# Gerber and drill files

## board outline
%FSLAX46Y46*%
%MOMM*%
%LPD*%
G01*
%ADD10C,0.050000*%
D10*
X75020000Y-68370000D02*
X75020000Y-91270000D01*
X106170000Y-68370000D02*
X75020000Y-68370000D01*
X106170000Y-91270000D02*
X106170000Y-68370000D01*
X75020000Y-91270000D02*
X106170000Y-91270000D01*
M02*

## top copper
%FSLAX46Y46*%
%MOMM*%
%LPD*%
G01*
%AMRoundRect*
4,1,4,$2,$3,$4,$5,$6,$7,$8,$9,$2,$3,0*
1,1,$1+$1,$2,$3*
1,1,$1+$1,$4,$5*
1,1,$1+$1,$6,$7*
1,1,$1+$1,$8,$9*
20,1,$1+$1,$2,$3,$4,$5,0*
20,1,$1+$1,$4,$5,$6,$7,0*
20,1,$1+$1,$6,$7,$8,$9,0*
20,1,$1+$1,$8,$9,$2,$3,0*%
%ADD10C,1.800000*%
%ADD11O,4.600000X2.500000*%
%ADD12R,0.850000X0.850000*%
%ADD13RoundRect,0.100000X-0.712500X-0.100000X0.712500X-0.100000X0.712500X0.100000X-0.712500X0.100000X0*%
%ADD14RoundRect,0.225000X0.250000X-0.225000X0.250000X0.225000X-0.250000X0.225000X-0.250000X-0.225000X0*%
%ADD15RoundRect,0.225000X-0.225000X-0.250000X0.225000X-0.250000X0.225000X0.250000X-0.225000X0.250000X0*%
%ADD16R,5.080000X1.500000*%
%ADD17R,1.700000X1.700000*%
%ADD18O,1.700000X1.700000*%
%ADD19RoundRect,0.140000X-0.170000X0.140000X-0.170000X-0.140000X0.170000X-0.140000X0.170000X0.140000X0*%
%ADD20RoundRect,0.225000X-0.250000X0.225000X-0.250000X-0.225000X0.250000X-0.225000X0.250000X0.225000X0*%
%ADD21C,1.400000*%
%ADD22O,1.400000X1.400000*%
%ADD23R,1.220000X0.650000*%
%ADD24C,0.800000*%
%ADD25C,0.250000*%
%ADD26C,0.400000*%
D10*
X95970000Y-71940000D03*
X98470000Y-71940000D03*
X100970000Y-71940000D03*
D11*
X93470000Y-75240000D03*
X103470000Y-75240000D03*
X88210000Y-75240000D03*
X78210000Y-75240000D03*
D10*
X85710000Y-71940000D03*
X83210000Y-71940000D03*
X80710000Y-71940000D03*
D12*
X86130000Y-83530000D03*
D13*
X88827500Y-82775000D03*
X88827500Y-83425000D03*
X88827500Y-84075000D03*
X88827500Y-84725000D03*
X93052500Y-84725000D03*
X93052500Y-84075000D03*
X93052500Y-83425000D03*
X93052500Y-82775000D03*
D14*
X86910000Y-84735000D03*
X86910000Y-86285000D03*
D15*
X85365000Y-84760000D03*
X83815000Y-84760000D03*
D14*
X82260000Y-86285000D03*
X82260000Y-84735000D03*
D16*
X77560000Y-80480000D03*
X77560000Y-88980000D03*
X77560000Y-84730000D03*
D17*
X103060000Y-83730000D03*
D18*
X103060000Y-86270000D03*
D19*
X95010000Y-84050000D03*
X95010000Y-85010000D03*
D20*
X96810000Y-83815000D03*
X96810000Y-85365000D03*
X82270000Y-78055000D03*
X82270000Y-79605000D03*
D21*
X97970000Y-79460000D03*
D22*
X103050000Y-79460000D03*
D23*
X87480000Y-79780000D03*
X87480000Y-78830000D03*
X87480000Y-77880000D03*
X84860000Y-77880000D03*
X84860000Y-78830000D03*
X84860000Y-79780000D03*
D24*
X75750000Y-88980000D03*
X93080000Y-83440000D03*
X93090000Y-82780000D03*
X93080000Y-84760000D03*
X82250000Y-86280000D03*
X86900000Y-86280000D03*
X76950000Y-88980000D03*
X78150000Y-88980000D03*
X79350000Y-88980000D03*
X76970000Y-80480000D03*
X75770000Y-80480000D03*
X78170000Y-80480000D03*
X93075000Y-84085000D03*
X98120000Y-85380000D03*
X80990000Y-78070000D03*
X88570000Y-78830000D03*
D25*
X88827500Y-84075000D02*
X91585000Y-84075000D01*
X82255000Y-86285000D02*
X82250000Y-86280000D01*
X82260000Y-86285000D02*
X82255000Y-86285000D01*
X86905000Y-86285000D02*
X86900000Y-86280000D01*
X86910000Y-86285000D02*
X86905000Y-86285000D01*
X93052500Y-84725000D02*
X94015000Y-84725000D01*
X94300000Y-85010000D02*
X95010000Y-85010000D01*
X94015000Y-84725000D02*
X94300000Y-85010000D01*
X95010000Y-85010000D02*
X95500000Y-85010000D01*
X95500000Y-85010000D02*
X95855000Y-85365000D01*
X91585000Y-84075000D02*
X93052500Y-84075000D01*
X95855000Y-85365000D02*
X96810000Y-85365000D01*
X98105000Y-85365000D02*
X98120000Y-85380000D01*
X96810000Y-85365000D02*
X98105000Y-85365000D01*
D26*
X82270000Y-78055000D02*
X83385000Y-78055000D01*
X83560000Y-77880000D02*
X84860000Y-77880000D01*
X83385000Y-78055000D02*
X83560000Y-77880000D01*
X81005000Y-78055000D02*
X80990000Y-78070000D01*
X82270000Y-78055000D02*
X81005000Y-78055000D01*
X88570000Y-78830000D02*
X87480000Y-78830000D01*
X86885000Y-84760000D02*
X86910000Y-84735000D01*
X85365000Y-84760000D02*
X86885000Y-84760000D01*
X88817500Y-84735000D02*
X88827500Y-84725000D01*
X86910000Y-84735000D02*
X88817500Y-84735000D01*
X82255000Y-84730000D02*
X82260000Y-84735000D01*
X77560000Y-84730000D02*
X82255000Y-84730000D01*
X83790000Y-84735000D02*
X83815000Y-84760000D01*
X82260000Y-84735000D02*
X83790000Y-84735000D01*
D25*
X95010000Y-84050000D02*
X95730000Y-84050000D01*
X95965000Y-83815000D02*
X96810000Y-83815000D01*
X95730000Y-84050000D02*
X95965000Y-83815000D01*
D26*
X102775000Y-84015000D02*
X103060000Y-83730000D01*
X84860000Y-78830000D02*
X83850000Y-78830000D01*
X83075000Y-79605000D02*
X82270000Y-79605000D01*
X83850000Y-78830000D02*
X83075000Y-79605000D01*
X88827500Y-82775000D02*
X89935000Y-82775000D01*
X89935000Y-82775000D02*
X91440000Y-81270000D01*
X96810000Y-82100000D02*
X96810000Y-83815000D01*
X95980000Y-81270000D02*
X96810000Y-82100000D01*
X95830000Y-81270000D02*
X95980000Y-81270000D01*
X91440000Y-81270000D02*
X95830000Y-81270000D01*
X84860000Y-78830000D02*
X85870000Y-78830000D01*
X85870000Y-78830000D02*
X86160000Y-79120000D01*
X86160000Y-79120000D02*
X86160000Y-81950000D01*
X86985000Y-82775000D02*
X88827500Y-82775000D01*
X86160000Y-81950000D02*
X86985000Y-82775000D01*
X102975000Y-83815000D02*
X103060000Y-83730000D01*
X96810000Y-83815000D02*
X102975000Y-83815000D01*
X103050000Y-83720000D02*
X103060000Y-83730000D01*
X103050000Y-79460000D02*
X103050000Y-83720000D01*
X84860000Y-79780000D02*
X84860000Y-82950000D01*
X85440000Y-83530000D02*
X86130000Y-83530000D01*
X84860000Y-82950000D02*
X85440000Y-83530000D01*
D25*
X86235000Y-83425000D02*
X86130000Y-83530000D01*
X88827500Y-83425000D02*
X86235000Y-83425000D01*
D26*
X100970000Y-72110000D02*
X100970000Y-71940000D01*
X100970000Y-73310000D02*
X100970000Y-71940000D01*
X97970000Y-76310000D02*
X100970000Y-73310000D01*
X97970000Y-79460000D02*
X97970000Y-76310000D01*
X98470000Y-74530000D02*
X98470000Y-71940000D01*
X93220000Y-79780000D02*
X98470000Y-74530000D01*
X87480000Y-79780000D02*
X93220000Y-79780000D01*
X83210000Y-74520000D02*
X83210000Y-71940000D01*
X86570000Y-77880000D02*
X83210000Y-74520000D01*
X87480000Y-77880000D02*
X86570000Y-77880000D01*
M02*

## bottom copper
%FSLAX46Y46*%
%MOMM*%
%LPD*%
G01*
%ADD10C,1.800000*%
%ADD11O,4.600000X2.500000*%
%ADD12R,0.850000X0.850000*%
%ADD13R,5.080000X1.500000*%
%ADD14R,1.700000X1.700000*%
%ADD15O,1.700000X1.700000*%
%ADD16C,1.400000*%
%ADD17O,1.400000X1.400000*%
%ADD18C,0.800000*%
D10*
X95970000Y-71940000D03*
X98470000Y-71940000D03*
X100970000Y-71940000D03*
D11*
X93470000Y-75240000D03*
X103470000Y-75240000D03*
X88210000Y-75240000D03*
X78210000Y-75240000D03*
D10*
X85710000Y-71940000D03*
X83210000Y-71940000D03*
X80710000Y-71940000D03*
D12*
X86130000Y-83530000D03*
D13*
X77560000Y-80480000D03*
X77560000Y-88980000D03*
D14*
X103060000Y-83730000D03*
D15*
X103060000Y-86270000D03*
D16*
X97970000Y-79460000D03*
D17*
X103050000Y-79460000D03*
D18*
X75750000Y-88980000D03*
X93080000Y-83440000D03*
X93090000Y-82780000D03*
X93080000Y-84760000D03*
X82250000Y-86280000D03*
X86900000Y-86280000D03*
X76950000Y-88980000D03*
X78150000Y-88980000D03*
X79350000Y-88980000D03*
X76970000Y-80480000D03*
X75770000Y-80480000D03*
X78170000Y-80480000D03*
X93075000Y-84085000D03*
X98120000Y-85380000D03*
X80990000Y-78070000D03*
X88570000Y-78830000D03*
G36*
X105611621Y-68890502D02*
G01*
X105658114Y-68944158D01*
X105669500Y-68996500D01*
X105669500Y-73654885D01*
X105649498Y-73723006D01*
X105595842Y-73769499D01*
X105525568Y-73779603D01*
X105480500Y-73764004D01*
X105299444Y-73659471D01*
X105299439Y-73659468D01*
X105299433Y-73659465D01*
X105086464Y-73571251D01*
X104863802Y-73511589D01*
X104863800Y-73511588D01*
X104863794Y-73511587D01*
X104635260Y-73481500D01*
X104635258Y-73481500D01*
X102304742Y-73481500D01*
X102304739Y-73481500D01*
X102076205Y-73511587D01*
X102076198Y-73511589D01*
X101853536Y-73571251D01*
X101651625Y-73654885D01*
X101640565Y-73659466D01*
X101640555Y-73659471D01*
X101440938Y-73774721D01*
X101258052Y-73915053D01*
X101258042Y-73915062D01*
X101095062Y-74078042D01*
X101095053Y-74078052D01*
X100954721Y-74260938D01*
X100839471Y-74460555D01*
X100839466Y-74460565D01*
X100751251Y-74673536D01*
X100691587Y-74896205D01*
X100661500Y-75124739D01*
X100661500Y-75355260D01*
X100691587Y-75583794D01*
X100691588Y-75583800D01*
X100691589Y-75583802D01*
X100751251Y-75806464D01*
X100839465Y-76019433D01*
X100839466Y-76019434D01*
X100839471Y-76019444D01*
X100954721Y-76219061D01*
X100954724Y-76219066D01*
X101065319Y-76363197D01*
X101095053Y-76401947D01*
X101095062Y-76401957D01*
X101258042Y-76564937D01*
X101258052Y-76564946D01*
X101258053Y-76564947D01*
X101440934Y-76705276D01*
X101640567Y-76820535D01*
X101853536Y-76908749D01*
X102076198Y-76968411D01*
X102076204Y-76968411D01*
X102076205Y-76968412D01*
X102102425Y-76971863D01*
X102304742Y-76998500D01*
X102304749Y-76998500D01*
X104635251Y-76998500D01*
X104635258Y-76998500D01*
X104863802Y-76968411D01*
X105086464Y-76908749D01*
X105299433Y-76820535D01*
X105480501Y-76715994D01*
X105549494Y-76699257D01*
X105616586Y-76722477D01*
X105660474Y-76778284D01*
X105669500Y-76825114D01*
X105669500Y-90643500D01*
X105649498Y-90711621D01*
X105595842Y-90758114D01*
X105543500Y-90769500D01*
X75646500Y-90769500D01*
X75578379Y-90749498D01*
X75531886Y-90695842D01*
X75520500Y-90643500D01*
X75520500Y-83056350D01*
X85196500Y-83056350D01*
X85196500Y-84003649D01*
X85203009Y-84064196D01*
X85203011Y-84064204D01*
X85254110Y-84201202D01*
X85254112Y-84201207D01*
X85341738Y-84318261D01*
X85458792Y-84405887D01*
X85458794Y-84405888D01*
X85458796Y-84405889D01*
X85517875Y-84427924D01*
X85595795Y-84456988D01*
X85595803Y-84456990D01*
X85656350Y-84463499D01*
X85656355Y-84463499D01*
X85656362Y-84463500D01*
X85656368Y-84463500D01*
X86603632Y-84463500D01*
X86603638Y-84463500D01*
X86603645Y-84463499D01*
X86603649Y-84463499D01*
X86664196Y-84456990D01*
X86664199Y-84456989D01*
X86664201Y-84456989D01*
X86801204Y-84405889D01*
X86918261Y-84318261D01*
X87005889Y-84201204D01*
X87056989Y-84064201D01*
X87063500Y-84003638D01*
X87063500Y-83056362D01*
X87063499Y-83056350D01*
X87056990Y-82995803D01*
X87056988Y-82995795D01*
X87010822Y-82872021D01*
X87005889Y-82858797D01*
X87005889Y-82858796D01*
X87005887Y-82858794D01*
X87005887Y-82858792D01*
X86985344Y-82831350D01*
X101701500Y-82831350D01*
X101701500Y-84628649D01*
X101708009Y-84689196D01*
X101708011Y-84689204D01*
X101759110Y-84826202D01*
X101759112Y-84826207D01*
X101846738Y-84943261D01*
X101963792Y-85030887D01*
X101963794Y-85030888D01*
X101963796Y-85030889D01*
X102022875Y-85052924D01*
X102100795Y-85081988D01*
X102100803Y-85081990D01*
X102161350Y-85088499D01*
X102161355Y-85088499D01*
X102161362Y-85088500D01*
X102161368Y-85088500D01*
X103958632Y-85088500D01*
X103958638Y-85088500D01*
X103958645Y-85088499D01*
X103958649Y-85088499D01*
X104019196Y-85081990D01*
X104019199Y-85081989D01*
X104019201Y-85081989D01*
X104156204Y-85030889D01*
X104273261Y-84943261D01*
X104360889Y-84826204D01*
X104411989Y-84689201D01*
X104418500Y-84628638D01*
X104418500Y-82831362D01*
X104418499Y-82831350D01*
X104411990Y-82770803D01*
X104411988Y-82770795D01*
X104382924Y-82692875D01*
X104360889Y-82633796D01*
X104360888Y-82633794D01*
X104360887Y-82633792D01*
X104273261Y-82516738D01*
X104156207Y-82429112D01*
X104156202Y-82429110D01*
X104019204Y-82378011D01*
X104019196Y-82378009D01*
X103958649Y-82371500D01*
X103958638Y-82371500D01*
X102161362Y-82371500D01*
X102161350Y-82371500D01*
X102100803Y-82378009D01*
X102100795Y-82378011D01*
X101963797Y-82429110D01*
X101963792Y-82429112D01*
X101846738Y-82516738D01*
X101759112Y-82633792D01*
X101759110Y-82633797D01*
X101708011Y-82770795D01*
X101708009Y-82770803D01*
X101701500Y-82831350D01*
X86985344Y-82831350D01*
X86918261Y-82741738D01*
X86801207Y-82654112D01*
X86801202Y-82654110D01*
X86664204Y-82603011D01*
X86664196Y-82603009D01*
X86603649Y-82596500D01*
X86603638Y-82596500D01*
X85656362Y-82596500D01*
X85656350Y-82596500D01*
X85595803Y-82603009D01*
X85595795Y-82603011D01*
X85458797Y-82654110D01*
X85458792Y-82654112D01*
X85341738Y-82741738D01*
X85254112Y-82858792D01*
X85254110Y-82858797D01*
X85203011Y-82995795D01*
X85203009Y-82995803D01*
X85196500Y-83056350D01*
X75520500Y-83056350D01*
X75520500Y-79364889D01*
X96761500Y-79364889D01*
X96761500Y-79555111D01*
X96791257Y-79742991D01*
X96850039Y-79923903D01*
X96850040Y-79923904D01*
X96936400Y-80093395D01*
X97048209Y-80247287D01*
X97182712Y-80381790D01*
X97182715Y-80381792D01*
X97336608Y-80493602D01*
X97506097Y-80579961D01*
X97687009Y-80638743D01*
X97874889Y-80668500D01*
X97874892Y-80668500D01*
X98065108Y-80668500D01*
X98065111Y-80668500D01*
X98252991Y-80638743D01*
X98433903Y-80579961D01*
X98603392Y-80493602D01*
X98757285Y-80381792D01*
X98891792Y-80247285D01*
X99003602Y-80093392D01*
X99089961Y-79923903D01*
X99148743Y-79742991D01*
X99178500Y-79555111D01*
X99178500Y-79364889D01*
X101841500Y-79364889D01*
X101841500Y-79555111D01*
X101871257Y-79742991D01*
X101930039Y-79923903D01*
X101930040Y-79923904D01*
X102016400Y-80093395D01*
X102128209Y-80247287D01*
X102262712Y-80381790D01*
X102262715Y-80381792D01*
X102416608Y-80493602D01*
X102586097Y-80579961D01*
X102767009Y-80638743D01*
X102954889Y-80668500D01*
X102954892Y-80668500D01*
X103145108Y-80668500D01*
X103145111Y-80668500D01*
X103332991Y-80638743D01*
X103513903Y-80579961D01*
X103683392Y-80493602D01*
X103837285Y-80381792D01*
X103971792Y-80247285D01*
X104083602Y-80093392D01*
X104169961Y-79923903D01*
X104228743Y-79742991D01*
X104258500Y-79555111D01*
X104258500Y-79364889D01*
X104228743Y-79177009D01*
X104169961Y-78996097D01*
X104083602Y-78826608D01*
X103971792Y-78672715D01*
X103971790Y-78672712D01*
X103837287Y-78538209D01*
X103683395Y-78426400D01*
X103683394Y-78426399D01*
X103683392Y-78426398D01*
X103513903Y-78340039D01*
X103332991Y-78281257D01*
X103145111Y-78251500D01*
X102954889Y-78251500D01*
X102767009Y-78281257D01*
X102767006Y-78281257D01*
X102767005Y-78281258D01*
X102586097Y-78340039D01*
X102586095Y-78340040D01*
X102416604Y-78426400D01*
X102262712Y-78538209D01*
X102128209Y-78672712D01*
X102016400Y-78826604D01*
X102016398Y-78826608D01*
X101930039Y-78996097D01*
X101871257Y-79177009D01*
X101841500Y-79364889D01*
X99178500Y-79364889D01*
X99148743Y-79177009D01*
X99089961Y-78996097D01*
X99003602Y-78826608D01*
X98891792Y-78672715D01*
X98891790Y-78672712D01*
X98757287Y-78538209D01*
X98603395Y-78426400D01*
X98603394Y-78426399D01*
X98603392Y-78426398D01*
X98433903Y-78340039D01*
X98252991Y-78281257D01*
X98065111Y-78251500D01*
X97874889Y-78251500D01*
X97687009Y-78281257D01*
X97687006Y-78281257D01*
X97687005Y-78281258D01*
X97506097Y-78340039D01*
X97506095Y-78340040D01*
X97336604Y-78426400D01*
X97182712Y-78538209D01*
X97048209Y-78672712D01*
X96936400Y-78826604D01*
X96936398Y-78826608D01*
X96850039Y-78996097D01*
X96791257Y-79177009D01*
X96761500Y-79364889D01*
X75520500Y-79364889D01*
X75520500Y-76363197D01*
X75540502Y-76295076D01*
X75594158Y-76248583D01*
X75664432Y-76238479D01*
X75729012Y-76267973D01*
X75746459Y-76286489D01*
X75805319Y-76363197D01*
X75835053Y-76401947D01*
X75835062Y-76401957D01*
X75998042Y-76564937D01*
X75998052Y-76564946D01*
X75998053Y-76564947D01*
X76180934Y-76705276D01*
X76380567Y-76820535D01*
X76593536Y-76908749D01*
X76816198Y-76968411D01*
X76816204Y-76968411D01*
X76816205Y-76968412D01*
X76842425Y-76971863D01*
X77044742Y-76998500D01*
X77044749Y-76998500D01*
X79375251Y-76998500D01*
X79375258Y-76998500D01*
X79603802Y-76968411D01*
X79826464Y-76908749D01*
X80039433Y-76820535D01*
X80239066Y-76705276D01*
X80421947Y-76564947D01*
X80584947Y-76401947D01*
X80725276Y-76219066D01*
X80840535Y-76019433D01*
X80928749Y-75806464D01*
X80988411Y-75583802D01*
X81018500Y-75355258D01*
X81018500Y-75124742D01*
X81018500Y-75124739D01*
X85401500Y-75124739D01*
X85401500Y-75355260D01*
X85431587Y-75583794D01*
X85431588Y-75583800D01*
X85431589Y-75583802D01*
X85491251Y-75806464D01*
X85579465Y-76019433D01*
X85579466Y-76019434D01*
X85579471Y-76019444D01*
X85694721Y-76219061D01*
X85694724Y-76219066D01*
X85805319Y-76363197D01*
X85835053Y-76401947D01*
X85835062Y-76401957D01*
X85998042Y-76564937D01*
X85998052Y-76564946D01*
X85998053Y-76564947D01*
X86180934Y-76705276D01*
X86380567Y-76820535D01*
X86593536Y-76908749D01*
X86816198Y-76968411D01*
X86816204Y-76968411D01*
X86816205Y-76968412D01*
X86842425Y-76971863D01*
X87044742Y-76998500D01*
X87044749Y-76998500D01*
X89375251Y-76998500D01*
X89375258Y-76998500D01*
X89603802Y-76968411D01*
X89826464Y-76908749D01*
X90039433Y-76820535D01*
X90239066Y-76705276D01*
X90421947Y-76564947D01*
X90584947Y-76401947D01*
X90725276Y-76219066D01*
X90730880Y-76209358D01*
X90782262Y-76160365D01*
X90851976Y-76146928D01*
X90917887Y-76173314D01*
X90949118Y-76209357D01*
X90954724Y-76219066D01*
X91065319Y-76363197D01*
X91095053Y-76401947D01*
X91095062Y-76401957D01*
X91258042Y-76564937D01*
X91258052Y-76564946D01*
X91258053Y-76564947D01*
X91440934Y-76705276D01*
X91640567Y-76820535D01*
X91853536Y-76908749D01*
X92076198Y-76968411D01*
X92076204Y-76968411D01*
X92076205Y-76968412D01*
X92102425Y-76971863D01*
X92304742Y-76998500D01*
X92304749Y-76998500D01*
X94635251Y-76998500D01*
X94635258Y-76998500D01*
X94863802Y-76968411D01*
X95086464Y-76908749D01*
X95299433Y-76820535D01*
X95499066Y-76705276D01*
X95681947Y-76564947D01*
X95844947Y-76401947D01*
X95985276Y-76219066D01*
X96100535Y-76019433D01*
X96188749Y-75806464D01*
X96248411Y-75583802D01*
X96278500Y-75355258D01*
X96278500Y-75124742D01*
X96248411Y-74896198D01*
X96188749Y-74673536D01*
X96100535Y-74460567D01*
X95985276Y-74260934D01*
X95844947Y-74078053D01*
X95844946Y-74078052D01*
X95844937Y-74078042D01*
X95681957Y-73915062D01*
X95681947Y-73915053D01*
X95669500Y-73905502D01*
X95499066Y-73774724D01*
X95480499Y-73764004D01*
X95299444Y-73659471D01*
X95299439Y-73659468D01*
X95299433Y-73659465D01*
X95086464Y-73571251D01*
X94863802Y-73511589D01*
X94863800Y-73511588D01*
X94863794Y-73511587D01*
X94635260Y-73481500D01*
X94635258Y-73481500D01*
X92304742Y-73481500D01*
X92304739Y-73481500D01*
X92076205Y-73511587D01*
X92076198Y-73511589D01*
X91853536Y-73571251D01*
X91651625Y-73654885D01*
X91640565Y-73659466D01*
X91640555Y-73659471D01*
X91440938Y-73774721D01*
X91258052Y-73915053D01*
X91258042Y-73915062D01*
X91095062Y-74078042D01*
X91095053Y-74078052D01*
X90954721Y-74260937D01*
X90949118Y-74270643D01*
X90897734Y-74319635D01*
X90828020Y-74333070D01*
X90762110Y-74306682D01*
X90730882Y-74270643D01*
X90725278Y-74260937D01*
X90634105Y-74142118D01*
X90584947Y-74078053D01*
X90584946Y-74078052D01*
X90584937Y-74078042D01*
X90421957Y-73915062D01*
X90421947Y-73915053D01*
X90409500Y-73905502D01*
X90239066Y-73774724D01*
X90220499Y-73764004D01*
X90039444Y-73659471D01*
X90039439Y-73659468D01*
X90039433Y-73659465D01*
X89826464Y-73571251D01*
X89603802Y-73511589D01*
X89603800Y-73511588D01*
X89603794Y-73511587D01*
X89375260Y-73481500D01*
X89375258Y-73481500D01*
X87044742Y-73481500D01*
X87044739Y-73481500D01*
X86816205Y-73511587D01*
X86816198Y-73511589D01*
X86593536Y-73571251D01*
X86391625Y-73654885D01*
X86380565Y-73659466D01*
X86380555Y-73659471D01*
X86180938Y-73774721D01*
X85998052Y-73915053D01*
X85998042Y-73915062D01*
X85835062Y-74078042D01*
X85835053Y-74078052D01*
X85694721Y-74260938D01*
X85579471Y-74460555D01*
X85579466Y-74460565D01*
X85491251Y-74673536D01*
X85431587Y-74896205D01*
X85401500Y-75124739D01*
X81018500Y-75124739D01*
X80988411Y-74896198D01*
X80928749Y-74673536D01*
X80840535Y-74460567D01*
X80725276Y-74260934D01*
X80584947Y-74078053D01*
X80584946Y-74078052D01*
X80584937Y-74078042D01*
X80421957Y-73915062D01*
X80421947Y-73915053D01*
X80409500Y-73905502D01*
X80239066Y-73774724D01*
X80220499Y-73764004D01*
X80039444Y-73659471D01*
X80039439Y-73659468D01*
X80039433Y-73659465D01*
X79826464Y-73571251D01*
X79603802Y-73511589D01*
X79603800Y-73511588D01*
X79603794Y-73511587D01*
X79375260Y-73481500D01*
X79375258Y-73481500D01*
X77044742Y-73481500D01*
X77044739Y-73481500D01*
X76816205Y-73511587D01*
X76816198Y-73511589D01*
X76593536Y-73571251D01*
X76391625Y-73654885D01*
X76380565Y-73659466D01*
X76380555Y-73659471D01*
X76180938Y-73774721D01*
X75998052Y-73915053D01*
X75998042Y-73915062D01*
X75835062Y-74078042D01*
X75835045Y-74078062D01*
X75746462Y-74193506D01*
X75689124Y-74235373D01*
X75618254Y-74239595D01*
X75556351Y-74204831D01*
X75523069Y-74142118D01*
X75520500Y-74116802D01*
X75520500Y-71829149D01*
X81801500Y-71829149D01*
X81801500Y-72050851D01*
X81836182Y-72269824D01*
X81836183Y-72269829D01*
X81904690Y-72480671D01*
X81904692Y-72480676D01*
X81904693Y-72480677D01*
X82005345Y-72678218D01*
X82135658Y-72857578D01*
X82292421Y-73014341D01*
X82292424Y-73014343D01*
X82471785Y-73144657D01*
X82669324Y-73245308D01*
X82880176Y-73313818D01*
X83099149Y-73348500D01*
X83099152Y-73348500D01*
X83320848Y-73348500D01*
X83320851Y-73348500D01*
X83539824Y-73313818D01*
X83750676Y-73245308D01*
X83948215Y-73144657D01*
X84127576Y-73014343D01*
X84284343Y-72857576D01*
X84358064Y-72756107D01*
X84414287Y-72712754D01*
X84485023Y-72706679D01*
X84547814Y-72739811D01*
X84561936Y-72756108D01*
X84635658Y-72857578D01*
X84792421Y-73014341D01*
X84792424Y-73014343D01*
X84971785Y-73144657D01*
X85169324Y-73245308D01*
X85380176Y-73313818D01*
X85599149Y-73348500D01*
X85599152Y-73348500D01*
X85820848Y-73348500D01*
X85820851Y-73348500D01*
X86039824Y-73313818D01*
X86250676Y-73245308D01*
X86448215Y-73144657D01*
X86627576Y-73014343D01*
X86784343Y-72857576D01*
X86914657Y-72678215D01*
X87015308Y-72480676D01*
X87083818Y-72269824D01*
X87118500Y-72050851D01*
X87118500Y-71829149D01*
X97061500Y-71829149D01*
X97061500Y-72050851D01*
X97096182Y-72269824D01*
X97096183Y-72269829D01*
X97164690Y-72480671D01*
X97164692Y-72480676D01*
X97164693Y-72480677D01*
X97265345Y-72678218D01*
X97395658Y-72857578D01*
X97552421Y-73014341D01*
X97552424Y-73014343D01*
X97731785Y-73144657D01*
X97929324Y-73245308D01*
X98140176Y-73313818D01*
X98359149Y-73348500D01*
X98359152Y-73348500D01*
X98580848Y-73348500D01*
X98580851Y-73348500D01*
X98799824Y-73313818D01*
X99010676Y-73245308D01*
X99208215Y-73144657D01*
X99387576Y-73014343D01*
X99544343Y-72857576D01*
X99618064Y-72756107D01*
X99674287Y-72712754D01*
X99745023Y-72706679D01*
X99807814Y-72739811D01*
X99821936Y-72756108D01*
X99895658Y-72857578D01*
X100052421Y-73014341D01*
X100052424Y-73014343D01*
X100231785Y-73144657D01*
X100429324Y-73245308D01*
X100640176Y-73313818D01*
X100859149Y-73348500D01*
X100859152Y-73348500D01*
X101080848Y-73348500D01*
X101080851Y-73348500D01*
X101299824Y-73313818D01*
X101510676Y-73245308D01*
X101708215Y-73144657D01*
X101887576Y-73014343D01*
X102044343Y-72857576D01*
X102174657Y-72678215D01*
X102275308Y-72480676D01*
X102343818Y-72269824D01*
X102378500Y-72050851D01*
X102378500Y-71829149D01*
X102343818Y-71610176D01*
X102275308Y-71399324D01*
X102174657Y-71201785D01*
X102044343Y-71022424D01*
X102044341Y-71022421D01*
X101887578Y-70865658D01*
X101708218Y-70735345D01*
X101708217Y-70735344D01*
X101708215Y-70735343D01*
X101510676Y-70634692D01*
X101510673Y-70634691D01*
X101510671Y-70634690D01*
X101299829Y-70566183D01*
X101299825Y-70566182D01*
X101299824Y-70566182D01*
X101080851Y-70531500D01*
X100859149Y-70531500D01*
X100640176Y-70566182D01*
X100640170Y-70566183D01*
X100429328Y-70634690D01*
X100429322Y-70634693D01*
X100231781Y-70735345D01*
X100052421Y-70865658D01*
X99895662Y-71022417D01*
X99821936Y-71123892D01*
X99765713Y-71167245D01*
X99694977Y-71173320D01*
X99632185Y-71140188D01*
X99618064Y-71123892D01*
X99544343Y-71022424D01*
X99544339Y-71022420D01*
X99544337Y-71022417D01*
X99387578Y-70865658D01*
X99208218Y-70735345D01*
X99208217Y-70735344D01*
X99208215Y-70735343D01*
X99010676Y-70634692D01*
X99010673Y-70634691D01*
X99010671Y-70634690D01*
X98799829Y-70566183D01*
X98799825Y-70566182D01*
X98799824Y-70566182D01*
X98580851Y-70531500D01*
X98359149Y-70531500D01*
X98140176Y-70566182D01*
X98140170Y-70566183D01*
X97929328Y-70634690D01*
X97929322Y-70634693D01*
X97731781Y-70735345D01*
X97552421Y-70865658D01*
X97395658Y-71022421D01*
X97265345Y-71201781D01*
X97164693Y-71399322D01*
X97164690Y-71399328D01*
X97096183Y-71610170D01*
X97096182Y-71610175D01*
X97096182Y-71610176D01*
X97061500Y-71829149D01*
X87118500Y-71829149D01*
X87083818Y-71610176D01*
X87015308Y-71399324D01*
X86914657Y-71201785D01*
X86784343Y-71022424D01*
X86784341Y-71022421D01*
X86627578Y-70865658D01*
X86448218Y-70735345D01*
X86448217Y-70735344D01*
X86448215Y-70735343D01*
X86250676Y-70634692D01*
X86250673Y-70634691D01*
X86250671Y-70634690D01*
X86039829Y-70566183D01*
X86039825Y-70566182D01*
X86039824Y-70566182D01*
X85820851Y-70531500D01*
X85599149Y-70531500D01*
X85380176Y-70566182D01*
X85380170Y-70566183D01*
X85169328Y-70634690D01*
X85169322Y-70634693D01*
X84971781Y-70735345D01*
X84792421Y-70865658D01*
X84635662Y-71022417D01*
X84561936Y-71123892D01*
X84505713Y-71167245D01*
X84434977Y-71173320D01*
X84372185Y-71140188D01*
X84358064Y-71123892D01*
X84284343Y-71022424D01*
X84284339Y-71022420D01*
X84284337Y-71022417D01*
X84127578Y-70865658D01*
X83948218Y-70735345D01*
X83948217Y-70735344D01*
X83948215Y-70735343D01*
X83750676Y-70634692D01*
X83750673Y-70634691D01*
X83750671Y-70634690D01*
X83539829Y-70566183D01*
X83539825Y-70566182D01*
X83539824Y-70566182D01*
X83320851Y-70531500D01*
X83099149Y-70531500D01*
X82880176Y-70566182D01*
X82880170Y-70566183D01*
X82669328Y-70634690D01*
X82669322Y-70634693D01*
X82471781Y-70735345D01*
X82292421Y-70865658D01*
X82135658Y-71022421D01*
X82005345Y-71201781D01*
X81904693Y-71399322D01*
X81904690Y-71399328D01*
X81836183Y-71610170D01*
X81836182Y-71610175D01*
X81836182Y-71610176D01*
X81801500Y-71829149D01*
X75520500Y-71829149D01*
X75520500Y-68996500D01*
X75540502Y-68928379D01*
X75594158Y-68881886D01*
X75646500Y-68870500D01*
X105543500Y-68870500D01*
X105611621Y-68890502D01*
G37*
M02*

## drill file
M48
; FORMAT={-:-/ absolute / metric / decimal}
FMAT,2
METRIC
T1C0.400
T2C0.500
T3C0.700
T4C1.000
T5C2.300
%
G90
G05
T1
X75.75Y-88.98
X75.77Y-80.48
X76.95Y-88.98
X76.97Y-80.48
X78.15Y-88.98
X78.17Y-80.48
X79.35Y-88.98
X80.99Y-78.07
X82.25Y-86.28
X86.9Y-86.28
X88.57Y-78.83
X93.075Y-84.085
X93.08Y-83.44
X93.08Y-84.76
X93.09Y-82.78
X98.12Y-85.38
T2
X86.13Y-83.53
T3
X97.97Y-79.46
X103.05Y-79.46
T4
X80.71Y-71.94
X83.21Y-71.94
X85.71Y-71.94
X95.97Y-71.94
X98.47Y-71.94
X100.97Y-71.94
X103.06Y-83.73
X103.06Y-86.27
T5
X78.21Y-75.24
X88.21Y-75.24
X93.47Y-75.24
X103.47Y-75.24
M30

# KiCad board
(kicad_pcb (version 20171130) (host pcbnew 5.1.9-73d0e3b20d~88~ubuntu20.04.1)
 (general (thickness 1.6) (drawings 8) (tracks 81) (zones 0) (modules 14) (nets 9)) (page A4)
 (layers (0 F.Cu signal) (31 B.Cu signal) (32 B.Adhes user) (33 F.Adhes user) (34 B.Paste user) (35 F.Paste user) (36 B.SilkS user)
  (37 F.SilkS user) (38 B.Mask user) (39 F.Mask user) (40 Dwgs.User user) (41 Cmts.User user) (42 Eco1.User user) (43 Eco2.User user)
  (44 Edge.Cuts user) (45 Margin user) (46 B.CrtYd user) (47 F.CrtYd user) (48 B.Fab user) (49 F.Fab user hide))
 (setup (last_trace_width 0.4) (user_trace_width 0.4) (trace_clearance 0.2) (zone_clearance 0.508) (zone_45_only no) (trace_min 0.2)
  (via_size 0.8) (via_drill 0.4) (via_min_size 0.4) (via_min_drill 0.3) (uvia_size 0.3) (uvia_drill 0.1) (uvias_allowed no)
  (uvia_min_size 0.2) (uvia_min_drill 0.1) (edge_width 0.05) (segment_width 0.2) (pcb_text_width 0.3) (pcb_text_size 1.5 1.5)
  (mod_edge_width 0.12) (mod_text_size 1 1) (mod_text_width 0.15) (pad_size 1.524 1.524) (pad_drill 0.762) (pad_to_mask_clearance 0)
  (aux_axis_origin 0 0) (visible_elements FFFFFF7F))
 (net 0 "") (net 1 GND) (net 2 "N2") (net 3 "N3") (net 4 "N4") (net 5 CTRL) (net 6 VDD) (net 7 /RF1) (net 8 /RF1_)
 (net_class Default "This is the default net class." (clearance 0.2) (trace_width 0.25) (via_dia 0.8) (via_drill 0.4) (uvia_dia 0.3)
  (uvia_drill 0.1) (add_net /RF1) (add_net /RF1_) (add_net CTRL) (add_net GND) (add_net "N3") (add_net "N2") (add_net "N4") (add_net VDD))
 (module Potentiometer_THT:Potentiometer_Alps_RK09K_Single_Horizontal (layer F.Cu) (at 100.97 71.94 90)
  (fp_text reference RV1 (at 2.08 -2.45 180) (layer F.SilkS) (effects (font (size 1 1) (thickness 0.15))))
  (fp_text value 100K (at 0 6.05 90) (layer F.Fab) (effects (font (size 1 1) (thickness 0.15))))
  (pad 3 thru_hole circle (at 0 -5 90) (size 1.8 1.8) (drill 1) (layers *.Cu *.Mask) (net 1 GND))
  (pad 2 thru_hole circle (at 0 -2.5 90) (size 1.8 1.8) (drill 1) (layers *.Cu *.Mask) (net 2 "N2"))
  (pad 1 thru_hole circle (at 0 0 90) (size 1.8 1.8) (drill 1) (layers *.Cu *.Mask) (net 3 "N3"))
  (pad "" thru_hole oval (at -3.3 -7.5 90) (size 2.5 4.6) (drill 2.3) (layers *.Cu *.Mask))
  (pad "" thru_hole oval (at -3.3 2.5 90) (size 2.5 4.6) (drill 2.3) (layers *.Cu *.Mask)))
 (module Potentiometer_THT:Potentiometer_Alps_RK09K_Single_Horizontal (layer F.Cu) (at 85.71 71.94 90)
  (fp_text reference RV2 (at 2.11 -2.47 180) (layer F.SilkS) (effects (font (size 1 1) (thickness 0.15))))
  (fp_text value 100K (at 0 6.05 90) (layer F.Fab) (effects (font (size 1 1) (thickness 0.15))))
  (pad "" thru_hole oval (at -3.3 2.5 90) (size 2.5 4.6) (drill 2.3) (layers *.Cu *.Mask))
  (pad "" thru_hole oval (at -3.3 -7.5 90) (size 2.5 4.6) (drill 2.3) (layers *.Cu *.Mask))
  (pad 1 thru_hole circle (at 0 0 90) (size 1.8 1.8) (drill 1) (layers *.Cu *.Mask))
  (pad 2 thru_hole circle (at 0 -2.5 90) (size 1.8 1.8) (drill 1) (layers *.Cu *.Mask) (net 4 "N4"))
  (pad 3 thru_hole circle (at 0 -5 90) (size 1.8 1.8) (drill 1) (layers *.Cu *.Mask) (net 1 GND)))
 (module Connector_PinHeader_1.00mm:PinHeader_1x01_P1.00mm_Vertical (layer F.Cu) (at 86.13 83.53)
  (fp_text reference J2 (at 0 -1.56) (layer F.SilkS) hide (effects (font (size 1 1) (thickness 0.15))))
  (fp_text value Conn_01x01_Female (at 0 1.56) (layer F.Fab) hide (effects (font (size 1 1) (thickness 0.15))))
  (pad 1 thru_hole rect (at 0 0) (size 0.85 0.85) (drill 0.5) (layers *.Cu *.Mask) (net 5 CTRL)))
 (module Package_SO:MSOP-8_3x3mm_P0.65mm (layer F.Cu) (at 90.94 83.75)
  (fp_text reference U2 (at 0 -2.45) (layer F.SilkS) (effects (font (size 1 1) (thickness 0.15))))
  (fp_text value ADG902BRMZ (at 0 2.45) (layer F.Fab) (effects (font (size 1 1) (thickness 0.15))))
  (pad 1 smd roundrect (at -2.1125 -0.975) (size 1.625 0.4) (layers F.Cu F.Paste F.Mask) (roundrect_rratio 0.25) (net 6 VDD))
  (pad 2 smd roundrect (at -2.1125 -0.325) (size 1.625 0.4) (layers F.Cu F.Paste F.Mask) (roundrect_rratio 0.25) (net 5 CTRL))
  (pad 3 smd roundrect (at -2.1125 0.325) (size 1.625 0.4) (layers F.Cu F.Paste F.Mask) (roundrect_rratio 0.25) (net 1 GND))
  (pad 4 smd roundrect (at -2.1125 0.975) (size 1.625 0.4) (layers F.Cu F.Paste F.Mask) (roundrect_rratio 0.25) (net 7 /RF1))
  (pad 5 smd roundrect (at 2.1125 0.975) (size 1.625 0.4) (layers F.Cu F.Paste F.Mask) (roundrect_rratio 0.25) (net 1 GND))
  (pad 6 smd roundrect (at 2.1125 0.325) (size 1.625 0.4) (layers F.Cu F.Paste F.Mask) (roundrect_rratio 0.25) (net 1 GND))
  (pad 7 smd roundrect (at 2.1125 -0.325) (size 1.625 0.4) (layers F.Cu F.Paste F.Mask) (roundrect_rratio 0.25) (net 1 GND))
  (pad 8 smd roundrect (at 2.1125 -0.975) (size 1.625 0.4) (layers F.Cu F.Paste F.Mask) (roundrect_rratio 0.25) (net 1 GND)))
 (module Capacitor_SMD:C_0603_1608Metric (layer F.Cu) (at 86.91 85.51 90)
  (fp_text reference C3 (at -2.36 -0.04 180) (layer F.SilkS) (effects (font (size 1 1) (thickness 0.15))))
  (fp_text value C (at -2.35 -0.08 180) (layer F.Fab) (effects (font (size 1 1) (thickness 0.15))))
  (pad 2 smd roundrect (at 0.775 0 90) (size 0.9 0.95) (layers F.Cu F.Paste F.Mask) (roundrect_rratio 0.25) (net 7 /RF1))
  (pad 1 smd roundrect (at -0.775 0 90) (size 0.9 0.95) (layers F.Cu F.Paste F.Mask) (roundrect_rratio 0.25) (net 1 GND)))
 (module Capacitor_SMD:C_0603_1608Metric (layer F.Cu) (at 84.59 84.76)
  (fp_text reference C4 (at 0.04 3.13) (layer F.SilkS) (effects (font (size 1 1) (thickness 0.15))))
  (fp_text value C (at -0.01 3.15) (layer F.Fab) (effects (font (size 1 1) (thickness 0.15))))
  (pad 2 smd roundrect (at 0.775 0) (size 0.9 0.95) (layers F.Cu F.Paste F.Mask) (roundrect_rratio 0.25) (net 7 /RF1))
  (pad 1 smd roundrect (at -0.775 0) (size 0.9 0.95) (layers F.Cu F.Paste F.Mask) (roundrect_rratio 0.25) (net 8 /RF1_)))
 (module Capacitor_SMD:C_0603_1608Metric (layer F.Cu) (at 82.26 85.51 90)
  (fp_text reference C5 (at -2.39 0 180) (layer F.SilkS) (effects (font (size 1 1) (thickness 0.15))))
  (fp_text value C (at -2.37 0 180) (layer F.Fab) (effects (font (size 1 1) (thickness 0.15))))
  (pad 1 smd roundrect (at -0.775 0 90) (size 0.9 0.95) (layers F.Cu F.Paste F.Mask) (roundrect_rratio 0.25) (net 1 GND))
  (pad 2 smd roundrect (at 0.775 0 90) (size 0.9 0.95) (layers F.Cu F.Paste F.Mask) (roundrect_rratio 0.25) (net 8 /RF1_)))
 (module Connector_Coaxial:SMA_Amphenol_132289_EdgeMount (layer F.Cu) (at 77.56 84.73 180)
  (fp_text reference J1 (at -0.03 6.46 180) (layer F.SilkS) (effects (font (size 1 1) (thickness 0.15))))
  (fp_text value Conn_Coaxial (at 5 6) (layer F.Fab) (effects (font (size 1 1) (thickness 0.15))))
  (pad 2 smd rect (at 0 4.25 270) (size 1.5 5.08) (layers B.Cu B.Paste B.Mask) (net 1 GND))
  (pad 2 smd rect (at 0 -4.25 270) (size 1.5 5.08) (layers B.Cu B.Paste B.Mask) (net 1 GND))
  (pad 2 smd rect (at 0 4.25 270) (size 1.5 5.08) (layers F.Cu F.Paste F.Mask) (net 1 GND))
  (pad 2 smd rect (at 0 -4.25 270) (size 1.5 5.08) (layers F.Cu F.Paste F.Mask) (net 1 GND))
  (pad 1 smd rect (at 0 0 270) (size 1.5 5.08) (layers F.Cu F.Paste F.Mask) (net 8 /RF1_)))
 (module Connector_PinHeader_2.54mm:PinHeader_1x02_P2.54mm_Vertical (layer F.Cu) (at 103.06 83.73)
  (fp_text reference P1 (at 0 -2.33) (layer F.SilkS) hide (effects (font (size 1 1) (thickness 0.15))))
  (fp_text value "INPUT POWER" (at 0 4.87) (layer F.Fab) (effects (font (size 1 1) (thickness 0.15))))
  (pad 1 thru_hole rect (at 0 0) (size 1.7 1.7) (drill 1) (layers *.Cu *.Mask) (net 6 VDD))
  (pad 2 thru_hole oval (at 0 2.54) (size 1.7 1.7) (drill 1) (layers *.Cu *.Mask) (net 1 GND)))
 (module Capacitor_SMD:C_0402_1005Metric (layer F.Cu) (at 95.01 84.53 270)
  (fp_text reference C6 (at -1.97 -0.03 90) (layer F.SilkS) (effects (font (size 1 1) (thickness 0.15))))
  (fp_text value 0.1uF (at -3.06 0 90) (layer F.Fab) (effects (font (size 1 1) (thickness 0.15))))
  (pad 1 smd roundrect (at -0.48 0 270) (size 0.56 0.62) (layers F.Cu F.Paste F.Mask) (roundrect_rratio 0.25) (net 6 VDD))
  (pad 2 smd roundrect (at 0.48 0 270) (size 0.56 0.62) (layers F.Cu F.Paste F.Mask) (roundrect_rratio 0.25) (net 1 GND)))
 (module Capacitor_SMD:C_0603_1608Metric (layer F.Cu) (at 96.81 84.59 270)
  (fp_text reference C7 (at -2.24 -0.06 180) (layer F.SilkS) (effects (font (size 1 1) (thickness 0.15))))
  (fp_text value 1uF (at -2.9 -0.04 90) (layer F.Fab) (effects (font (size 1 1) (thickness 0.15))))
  (pad 1 smd roundrect (at -0.775 0 270) (size 0.9 0.95) (layers F.Cu F.Paste F.Mask) (roundrect_rratio 0.25) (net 6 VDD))
  (pad 2 smd roundrect (at 0.775 0 270) (size 0.9 0.95) (layers F.Cu F.Paste F.Mask) (roundrect_rratio 0.25) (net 1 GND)))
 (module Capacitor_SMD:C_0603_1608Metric (layer F.Cu) (at 82.27 78.83 270)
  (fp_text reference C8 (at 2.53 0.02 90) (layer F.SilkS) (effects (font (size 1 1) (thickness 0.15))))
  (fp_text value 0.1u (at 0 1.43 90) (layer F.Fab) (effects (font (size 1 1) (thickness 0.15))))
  (pad 1 smd roundrect (at -0.775 0 270) (size 0.9 0.95) (layers F.Cu F.Paste F.Mask) (roundrect_rratio 0.25) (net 1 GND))
  (pad 2 smd roundrect (at 0.775 0 270) (size 0.9 0.95) (layers F.Cu F.Paste F.Mask) (roundrect_rratio 0.25) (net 6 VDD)))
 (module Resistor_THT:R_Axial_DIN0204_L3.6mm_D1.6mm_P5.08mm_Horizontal (layer F.Cu) (at 97.97 79.46)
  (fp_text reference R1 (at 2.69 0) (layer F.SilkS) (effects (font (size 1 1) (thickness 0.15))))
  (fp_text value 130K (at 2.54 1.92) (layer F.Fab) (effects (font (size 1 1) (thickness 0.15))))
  (pad 1 thru_hole circle (at 0 0) (size 1.4 1.4) (drill 0.7) (layers *.Cu *.Mask) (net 3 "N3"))
  (pad 2 thru_hole oval (at 5.08 0) (size 1.4 1.4) (drill 0.7) (layers *.Cu *.Mask) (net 6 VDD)))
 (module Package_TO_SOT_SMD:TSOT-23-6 (layer F.Cu) (at 86.17 78.83 180)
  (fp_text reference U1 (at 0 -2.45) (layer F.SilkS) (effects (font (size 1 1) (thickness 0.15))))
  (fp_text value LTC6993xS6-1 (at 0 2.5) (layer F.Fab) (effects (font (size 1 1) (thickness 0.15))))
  (pad 1 smd rect (at -1.31 -0.95 180) (size 1.22 0.65) (layers F.Cu F.Paste F.Mask) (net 2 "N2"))
  (pad 2 smd rect (at -1.31 0 180) (size 1.22 0.65) (layers F.Cu F.Paste F.Mask) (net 1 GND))
  (pad 3 smd rect (at -1.31 0.95 180) (size 1.22 0.65) (layers F.Cu F.Paste F.Mask) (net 4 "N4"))
  (pad 4 smd rect (at 1.31 0.95 180) (size 1.22 0.65) (layers F.Cu F.Paste F.Mask) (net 1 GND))
  (pad 5 smd rect (at 1.31 0 180) (size 1.22 0.65) (layers F.Cu F.Paste F.Mask) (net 6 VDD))
  (pad 6 smd rect (at 1.31 -0.95 180) (size 1.22 0.65) (layers F.Cu F.Paste F.Mask) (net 5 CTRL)))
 (gr_line (start 75.02 68.37) (end 75.02 91.27) (layer Edge.Cuts) (width 0.05))
 (gr_line (start 106.17 68.37) (end 75.02 68.37) (layer Edge.Cuts) (width 0.05))
 (gr_line (start 106.17 91.27) (end 106.17 68.37) (layer Edge.Cuts) (width 0.05))
 (gr_line (start 75.02 91.27) (end 106.17 91.27) (layer Edge.Cuts) (width 0.05))
 (via (at 75.75 88.98) (size 0.8) (drill 0.4) (layers F.Cu B.Cu) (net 1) (status 30))
 (segment (start 88.8275 84.075) (end 91.585 84.075) (width 0.25) (layer F.Cu) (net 1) (status 10))
 (via (at 93.08 83.44) (size 0.8) (drill 0.4) (layers F.Cu B.Cu) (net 1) (status 30))
 (via (at 93.09 82.78) (size 0.8) (drill 0.4) (layers F.Cu B.Cu) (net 1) (status 30))
 (via (at 93.08 84.76) (size 0.8) (drill 0.4) (layers F.Cu B.Cu) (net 1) (status 30))
 (via (at 82.25 86.28) (size 0.8) (drill 0.4) (layers F.Cu B.Cu) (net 1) (status 30))
 (segment (start 82.255 86.285) (end 82.25 86.28) (width 0.25) (layer F.Cu) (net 1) (status 30))
 (segment (start 82.26 86.285) (end 82.255 86.285) (width 0.25) (layer F.Cu) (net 1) (status 30))
 (via (at 86.9 86.28) (size 0.8) (drill 0.4) (layers F.Cu B.Cu) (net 1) (status 30))
 (segment (start 86.905 86.285) (end 86.9 86.28) (width 0.25) (layer F.Cu) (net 1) (status 30))
 (segment (start 86.91 86.285) (end 86.905 86.285) (width 0.25) (layer F.Cu) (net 1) (status 30))
 (via (at 76.95 88.98) (size 0.8) (drill 0.4) (layers F.Cu B.Cu) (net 1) (status 30))
 (via (at 78.15 88.98) (size 0.8) (drill 0.4) (layers F.Cu B.Cu) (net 1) (status 30))
 (via (at 79.35 88.98) (size 0.8) (drill 0.4) (layers F.Cu B.Cu) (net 1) (status 30))
 (via (at 76.97 80.48) (size 0.8) (drill 0.4) (layers F.Cu B.Cu) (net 1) (status 30))
 (via (at 75.77 80.48) (size 0.8) (drill 0.4) (layers F.Cu B.Cu) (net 1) (status 30))
 (via (at 78.17 80.48) (size 0.8) (drill 0.4) (layers F.Cu B.Cu) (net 1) (status 30))
 (segment (start 93.0525 84.725) (end 94.015 84.725) (width 0.25) (layer F.Cu) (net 1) (status 10))
 (segment (start 94.3 85.01) (end 95.01 85.01) (width 0.25) (layer F.Cu) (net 1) (status 20))
 (segment (start 94.015 84.725) (end 94.3 85.01) (width 0.25) (layer F.Cu) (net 1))
 (segment (start 95.01 85.01) (end 95.5 85.01) (width 0.25) (layer F.Cu) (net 1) (status 10))
 (segment (start 95.5 85.01) (end 95.855 85.365) (width 0.25) (layer F.Cu) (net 1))
 (segment (start 91.585 84.075) (end 93.0525 84.075) (width 0.25) (layer F.Cu) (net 1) (status 20))
 (via (at 93.075 84.085) (size 0.8) (drill 0.4) (layers F.Cu B.Cu) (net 1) (status 30))
 (segment (start 95.855 85.365) (end 96.81 85.365) (width 0.25) (layer F.Cu) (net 1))
 (via (at 98.12 85.38) (size 0.8) (drill 0.4) (layers F.Cu B.Cu) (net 1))
 (segment (start 98.105 85.365) (end 98.12 85.38) (width 0.25) (layer F.Cu) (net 1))
 (segment (start 96.81 85.365) (end 98.105 85.365) (width 0.25) (layer F.Cu) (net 1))
 (segment (start 82.27 78.055) (end 83.385 78.055) (width 0.4) (layer F.Cu) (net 1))
 (segment (start 83.56 77.88) (end 84.86 77.88) (width 0.4) (layer F.Cu) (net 1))
 (segment (start 83.385 78.055) (end 83.56 77.88) (width 0.4) (layer F.Cu) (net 1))
 (via (at 80.99 78.07) (size 0.8) (drill 0.4) (layers F.Cu B.Cu) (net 1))
 (segment (start 81.005 78.055) (end 80.99 78.07) (width 0.4) (layer F.Cu) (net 1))
 (segment (start 82.27 78.055) (end 81.005 78.055) (width 0.4) (layer F.Cu) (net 1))
 (segment (start 88.57 78.83) (end 87.48 78.83) (width 0.4) (layer F.Cu) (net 1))
 (via (at 88.57 78.83) (size 0.8) (drill 0.4) (layers F.Cu B.Cu) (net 1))
 (segment (start 86.885 84.76) (end 86.91 84.735) (width 0.4) (layer F.Cu) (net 7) (status 30))
 (segment (start 85.365 84.76) (end 86.885 84.76) (width 0.4) (layer F.Cu) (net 7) (status 30))
 (segment (start 88.8175 84.735) (end 88.8275 84.725) (width 0.4) (layer F.Cu) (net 7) (status 30))
 (segment (start 86.91 84.735) (end 88.8175 84.735) (width 0.4) (layer F.Cu) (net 7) (status 30))
 (segment (start 82.255 84.73) (end 82.26 84.735) (width 0.4) (layer F.Cu) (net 8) (status 30))
 (segment (start 77.56 84.73) (end 82.255 84.73) (width 0.4) (layer F.Cu) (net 8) (status 30))
 (segment (start 83.79 84.735) (end 83.815 84.76) (width 0.4) (layer F.Cu) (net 8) (status 30))
 (segment (start 82.26 84.735) (end 83.79 84.735) (width 0.4) (layer F.Cu) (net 8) (status 30))
 (segment (start 95.01 84.05) (end 95.73 84.05) (width 0.25) (layer F.Cu) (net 6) (status 10))
 (segment (start 95.965 83.815) (end 96.81 83.815) (width 0.25) (layer F.Cu) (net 6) (status 20))
 (segment (start 95.73 84.05) (end 95.965 83.815) (width 0.25) (layer F.Cu) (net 6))
 (segment (start 102.775 84.015) (end 103.06 83.73) (width 0.4) (layer F.Cu) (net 6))
 (segment (start 84.86 78.83) (end 83.85 78.83) (width 0.4) (layer F.Cu) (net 6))
 (segment (start 83.075 79.605) (end 82.27 79.605) (width 0.4) (layer F.Cu) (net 6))
 (segment (start 83.85 78.83) (end 83.075 79.605) (width 0.4) (layer F.Cu) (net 6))
 (segment (start 88.8275 82.775) (end 89.935 82.775) (width 0.4) (layer F.Cu) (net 6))
 (segment (start 89.935 82.775) (end 91.44 81.27) (width 0.4) (layer F.Cu) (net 6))
 (segment (start 96.81 82.1) (end 96.81 83.815) (width 0.4) (layer F.Cu) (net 6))
 (segment (start 95.98 81.27) (end 96.81 82.1) (width 0.4) (layer F.Cu) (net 6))
 (segment (start 95.83 81.27) (end 95.98 81.27) (width 0.4) (layer F.Cu) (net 6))
 (segment (start 91.44 81.27) (end 95.83 81.27) (width 0.4) (layer F.Cu) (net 6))
 (segment (start 84.86 78.83) (end 85.87 78.83) (width 0.4) (layer F.Cu) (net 6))
 (segment (start 85.87 78.83) (end 86.16 79.12) (width 0.4) (layer F.Cu) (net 6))
 (segment (start 86.16 79.12) (end 86.16 81.95) (width 0.4) (layer F.Cu) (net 6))
 (segment (start 86.985 82.775) (end 88.8275 82.775) (width 0.4) (layer F.Cu) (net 6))
 (segment (start 86.16 81.95) (end 86.985 82.775) (width 0.4) (layer F.Cu) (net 6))
 (segment (start 102.975 83.815) (end 103.06 83.73) (width 0.4) (layer F.Cu) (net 6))
 (segment (start 96.81 83.815) (end 102.975 83.815) (width 0.4) (layer F.Cu) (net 6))
 (segment (start 103.05 83.72) (end 103.06 83.73) (width 0.4) (layer F.Cu) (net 6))
 (segment (start 103.05 79.46) (end 103.05 83.72) (width 0.4) (layer F.Cu) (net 6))
 (segment (start 84.86 79.78) (end 84.86 82.95) (width 0.4) (layer F.Cu) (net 5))
 (segment (start 85.44 83.53) (end 86.13 83.53) (width 0.4) (layer F.Cu) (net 5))
 (segment (start 84.86 82.95) (end 85.44 83.53) (width 0.4) (layer F.Cu) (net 5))
 (segment (start 86.235 83.425) (end 86.13 83.53) (width 0.25) (layer F.Cu) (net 5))
 (segment (start 88.8275 83.425) (end 86.235 83.425) (width 0.25) (layer F.Cu) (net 5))
 (segment (start 100.97 72.11) (end 100.97 71.94) (width 0.4) (layer F.Cu) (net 3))
 (segment (start 100.97 73.31) (end 100.97 71.94) (width 0.4) (layer F.Cu) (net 3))
 (segment (start 97.97 76.31) (end 100.97 73.31) (width 0.4) (layer F.Cu) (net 3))
 (segment (start 97.97 79.46) (end 97.97 76.31) (width 0.4) (layer F.Cu) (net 3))
 (segment (start 98.47 74.53) (end 98.47 71.94) (width 0.4) (layer F.Cu) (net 2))
 (segment (start 93.22 79.78) (end 98.47 74.53) (width 0.4) (layer F.Cu) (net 2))
 (segment (start 87.48 79.78) (end 93.22 79.78) (width 0.4) (layer F.Cu) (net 2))
 (segment (start 83.21 74.52) (end 83.21 71.94) (width 0.4) (layer F.Cu) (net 4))
 (segment (start 86.57 77.88) (end 83.21 74.52) (width 0.4) (layer F.Cu) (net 4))
 (segment (start 87.48 77.88) (end 86.57 77.88) (width 0.4) (layer F.Cu) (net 4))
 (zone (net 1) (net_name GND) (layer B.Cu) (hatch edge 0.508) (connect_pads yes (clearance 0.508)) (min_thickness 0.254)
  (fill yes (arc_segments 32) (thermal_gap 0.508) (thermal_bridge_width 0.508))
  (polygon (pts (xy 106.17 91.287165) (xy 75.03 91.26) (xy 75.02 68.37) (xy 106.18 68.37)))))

